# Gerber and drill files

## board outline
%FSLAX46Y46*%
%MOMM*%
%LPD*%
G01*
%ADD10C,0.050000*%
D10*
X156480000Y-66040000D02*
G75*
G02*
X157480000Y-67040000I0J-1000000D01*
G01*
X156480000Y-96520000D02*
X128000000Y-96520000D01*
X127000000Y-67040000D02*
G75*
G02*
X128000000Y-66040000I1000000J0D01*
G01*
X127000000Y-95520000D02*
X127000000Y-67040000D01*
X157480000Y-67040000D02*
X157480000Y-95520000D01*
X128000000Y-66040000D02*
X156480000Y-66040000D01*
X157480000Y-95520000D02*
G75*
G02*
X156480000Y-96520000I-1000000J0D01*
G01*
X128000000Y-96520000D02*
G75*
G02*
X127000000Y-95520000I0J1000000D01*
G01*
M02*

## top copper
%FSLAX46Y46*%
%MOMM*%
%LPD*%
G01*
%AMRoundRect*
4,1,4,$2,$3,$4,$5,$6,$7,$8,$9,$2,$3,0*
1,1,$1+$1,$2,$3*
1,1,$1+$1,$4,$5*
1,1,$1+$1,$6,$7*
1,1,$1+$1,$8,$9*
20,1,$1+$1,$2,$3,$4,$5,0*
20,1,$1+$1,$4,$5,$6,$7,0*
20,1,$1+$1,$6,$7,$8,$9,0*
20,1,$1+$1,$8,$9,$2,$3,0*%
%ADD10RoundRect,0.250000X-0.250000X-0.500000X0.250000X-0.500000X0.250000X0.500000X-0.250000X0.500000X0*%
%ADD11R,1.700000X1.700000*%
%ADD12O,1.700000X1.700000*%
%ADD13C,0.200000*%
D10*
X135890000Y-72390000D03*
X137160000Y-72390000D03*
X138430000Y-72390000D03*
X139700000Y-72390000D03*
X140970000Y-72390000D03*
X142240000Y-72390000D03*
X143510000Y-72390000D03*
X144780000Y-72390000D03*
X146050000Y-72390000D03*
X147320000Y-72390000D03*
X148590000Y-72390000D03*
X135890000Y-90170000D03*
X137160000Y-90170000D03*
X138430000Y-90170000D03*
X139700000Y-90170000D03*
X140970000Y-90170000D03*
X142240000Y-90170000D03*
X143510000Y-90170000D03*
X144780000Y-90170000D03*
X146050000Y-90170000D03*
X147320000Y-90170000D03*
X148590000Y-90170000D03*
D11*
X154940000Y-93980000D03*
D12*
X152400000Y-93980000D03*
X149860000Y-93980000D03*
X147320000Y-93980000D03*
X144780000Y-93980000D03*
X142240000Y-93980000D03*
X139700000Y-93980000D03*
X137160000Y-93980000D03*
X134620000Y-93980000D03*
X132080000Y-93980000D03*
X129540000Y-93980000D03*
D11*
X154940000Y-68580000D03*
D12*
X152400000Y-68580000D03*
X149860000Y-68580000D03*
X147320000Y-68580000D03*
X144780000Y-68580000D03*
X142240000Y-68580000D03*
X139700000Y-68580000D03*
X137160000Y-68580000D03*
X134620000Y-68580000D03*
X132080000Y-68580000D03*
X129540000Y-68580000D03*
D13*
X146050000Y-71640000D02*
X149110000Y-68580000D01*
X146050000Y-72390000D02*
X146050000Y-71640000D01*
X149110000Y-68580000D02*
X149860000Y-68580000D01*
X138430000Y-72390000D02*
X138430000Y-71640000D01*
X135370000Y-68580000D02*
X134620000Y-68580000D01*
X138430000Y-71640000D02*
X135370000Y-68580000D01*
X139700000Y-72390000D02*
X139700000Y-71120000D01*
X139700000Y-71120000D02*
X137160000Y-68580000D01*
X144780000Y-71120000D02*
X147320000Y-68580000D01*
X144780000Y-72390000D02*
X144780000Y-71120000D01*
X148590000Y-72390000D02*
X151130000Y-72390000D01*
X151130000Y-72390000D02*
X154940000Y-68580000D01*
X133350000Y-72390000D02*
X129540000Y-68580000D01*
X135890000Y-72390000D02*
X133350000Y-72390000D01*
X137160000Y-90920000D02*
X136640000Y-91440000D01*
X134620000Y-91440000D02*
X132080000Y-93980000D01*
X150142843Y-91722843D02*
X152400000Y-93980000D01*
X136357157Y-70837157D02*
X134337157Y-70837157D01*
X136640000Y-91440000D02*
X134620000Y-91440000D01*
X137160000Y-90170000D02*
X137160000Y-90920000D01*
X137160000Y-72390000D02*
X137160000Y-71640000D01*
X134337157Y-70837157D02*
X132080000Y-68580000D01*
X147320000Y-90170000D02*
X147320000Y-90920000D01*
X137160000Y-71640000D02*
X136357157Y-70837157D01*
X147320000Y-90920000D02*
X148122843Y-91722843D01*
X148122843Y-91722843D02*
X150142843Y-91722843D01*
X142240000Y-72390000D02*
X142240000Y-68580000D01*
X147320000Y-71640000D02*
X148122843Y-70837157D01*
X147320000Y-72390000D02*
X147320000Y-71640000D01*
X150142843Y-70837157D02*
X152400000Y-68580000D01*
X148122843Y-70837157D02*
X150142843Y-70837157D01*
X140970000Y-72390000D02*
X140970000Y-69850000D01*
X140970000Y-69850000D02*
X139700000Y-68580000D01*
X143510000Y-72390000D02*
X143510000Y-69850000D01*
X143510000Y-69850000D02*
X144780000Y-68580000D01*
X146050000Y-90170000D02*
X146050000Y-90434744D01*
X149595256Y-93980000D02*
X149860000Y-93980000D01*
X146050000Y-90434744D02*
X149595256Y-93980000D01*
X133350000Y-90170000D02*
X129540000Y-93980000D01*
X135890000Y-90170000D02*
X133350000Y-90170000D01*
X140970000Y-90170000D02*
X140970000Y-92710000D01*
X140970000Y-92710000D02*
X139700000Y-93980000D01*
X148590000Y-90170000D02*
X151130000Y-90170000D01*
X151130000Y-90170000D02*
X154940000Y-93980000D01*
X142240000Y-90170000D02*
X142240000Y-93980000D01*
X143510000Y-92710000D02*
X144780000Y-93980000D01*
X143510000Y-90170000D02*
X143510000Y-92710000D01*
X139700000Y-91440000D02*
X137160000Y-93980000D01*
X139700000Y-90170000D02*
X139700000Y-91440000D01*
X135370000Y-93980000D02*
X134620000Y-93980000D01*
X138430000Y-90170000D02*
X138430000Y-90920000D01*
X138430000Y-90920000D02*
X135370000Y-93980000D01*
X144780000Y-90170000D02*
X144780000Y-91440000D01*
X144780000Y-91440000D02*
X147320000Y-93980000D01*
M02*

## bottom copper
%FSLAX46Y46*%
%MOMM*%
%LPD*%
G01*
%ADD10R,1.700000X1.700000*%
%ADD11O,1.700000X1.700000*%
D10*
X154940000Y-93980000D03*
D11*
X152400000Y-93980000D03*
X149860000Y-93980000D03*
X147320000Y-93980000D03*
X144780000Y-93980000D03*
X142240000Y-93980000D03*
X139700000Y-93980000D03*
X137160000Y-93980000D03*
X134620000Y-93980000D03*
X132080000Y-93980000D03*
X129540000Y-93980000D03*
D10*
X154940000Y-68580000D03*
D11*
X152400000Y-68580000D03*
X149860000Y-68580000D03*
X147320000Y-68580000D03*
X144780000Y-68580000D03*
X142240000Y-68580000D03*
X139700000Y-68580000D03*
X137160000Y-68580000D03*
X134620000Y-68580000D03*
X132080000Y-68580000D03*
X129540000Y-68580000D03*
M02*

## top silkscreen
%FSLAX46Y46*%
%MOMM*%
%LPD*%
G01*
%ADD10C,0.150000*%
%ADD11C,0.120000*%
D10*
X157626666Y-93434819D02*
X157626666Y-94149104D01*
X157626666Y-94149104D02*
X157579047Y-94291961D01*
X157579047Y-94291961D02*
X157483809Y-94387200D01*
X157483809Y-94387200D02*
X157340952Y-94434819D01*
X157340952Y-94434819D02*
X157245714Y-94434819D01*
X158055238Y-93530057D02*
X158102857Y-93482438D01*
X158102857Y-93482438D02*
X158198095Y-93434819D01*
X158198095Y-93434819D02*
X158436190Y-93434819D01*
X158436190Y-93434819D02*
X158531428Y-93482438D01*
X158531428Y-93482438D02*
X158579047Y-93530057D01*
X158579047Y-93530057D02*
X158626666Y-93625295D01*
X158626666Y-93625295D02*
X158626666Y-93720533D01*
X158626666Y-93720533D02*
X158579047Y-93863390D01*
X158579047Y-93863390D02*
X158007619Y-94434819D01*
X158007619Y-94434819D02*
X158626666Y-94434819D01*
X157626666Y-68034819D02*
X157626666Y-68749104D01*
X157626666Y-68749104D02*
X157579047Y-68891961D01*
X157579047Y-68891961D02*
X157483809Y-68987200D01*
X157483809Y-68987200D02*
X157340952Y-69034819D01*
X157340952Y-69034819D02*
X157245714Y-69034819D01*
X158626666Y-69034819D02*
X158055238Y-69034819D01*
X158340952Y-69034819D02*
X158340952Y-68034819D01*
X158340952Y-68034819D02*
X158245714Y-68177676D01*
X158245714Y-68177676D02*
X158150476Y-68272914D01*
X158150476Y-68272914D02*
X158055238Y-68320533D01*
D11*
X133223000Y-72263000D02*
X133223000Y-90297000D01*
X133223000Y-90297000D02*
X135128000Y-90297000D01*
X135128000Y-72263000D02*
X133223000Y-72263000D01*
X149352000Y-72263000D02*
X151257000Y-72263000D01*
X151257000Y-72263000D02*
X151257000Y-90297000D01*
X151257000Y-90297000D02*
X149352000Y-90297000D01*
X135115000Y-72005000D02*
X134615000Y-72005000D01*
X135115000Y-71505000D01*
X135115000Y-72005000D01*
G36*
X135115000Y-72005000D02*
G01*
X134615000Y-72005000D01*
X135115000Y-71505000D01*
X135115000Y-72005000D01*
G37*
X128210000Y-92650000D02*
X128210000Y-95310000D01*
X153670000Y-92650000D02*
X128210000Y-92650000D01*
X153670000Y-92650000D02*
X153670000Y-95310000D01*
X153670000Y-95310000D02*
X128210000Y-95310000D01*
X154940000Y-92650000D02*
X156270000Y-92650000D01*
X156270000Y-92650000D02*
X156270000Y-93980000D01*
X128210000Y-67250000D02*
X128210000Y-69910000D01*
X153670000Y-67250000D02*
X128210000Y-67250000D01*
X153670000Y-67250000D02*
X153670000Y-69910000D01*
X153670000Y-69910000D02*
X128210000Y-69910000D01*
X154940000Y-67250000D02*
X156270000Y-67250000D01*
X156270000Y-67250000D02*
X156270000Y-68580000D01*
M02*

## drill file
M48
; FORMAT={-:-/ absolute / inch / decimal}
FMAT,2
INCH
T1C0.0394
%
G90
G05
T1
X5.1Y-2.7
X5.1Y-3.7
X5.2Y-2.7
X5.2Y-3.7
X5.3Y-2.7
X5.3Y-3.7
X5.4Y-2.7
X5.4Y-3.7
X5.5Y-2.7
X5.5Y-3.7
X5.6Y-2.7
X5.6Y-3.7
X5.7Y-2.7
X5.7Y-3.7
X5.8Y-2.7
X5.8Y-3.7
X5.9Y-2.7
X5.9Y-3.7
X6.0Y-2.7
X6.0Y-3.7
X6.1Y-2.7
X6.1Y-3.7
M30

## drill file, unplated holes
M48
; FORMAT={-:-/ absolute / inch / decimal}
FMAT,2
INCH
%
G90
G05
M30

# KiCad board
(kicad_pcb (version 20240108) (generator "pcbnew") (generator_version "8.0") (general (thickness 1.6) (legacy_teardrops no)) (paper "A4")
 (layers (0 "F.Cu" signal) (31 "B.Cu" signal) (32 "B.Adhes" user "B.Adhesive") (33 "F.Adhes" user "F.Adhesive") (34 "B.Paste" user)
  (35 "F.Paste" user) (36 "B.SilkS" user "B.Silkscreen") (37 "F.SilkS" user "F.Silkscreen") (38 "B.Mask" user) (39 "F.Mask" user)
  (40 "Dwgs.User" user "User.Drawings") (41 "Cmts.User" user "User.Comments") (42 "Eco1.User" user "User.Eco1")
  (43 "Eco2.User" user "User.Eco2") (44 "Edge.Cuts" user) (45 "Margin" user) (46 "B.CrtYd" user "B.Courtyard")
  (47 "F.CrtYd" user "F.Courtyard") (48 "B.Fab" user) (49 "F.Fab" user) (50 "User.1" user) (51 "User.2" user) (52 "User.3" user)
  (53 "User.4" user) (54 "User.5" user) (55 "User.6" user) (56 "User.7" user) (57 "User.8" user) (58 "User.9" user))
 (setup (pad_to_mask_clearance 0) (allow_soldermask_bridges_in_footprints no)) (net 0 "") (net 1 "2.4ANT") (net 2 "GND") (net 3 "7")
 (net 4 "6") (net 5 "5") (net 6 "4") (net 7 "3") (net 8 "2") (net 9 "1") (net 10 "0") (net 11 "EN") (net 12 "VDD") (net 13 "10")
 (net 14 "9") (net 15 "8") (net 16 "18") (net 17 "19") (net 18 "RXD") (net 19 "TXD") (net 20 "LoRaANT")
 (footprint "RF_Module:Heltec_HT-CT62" (layer "F.Cu") (at 142.24 81.28)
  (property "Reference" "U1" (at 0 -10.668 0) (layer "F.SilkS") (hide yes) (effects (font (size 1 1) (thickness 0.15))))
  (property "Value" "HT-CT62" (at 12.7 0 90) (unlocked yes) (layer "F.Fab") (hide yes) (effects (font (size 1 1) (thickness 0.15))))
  (fp_line (start -9.017 -9.017) (end -9.017 9.017) (stroke (width 0.12) (type default)) (layer "F.SilkS"))
  (fp_line (start -9.017 9.017) (end -7.112 9.017) (stroke (width 0.12) (type default)) (layer "F.SilkS"))
  (fp_line (start -7.112 -9.017) (end -9.017 -9.017) (stroke (width 0.12) (type default)) (layer "F.SilkS"))
  (fp_line (start 7.112 -9.017) (end 9.017 -9.017) (stroke (width 0.12) (type default)) (layer "F.SilkS"))
  (fp_line (start 9.017 -9.017) (end 9.017 9.017) (stroke (width 0.12) (type default)) (layer "F.SilkS"))
  (fp_line (start 9.017 9.017) (end 7.112 9.017) (stroke (width 0.12) (type default)) (layer "F.SilkS"))
  (fp_poly
   (pts (xy -7.125 -9.275) (xy -7.625 -9.275) (xy -7.125 -9.775) (xy -7.125 -9.275)) (stroke (width 0.12) (type solid)) (fill solid)
   (layer "F.SilkS"))
  (pad "1" smd roundrect (at -6.35 -8.89) (size 1 1.5) (layers "F.Cu" "F.Paste" "F.Mask") (roundrect_rratio 0.25) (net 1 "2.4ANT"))
  (pad "2" smd roundrect (at -5.08 -8.89) (size 1 1.5) (layers "F.Cu" "F.Paste" "F.Mask") (roundrect_rratio 0.25) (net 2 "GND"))
  (pad "3" smd roundrect (at -3.81 -8.89) (size 1 1.5) (layers "F.Cu" "F.Paste" "F.Mask") (roundrect_rratio 0.25) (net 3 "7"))
  (pad "4" smd roundrect (at -2.54 -8.89) (size 1 1.5) (layers "F.Cu" "F.Paste" "F.Mask") (roundrect_rratio 0.25) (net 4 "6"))
  (pad "5" smd roundrect (at -1.27 -8.89) (size 1 1.5) (layers "F.Cu" "F.Paste" "F.Mask") (roundrect_rratio 0.25) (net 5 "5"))
  (pad "6" smd roundrect (at 0 -8.89) (size 1 1.5) (layers "F.Cu" "F.Paste" "F.Mask") (roundrect_rratio 0.25) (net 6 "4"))
  (pad "7" smd roundrect (at 1.27 -8.89) (size 1 1.5) (layers "F.Cu" "F.Paste" "F.Mask") (roundrect_rratio 0.25) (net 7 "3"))
  (pad "8" smd roundrect (at 2.54 -8.89) (size 1 1.5) (layers "F.Cu" "F.Paste" "F.Mask") (roundrect_rratio 0.25) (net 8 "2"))
  (pad "9" smd roundrect (at 3.81 -8.89) (size 1 1.5) (layers "F.Cu" "F.Paste" "F.Mask") (roundrect_rratio 0.25) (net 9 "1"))
  (pad "10" smd roundrect (at 5.08 -8.89) (size 1 1.5) (layers "F.Cu" "F.Paste" "F.Mask") (roundrect_rratio 0.25) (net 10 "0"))
  (pad "11" smd roundrect (at 6.35 -8.89) (size 1 1.5) (layers "F.Cu" "F.Paste" "F.Mask") (roundrect_rratio 0.25) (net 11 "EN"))
  (pad "12" smd roundrect (at -6.35 8.89) (size 1 1.5) (layers "F.Cu" "F.Paste" "F.Mask") (roundrect_rratio 0.25) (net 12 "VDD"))
  (pad "13" smd roundrect (at -5.08 8.89) (size 1 1.5) (layers "F.Cu" "F.Paste" "F.Mask") (roundrect_rratio 0.25) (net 2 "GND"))
  (pad "14" smd roundrect (at -3.81 8.89) (size 1 1.5) (layers "F.Cu" "F.Paste" "F.Mask") (roundrect_rratio 0.25) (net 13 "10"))
  (pad "15" smd roundrect (at -2.54 8.89) (size 1 1.5) (layers "F.Cu" "F.Paste" "F.Mask") (roundrect_rratio 0.25) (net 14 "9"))
  (pad "16" smd roundrect (at -1.27 8.89) (size 1 1.5) (layers "F.Cu" "F.Paste" "F.Mask") (roundrect_rratio 0.25) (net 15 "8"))
  (pad "17" smd roundrect (at 0 8.89) (size 1 1.5) (layers "F.Cu" "F.Paste" "F.Mask") (roundrect_rratio 0.25) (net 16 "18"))
  (pad "18" smd roundrect (at 1.27 8.89) (size 1 1.5) (layers "F.Cu" "F.Paste" "F.Mask") (roundrect_rratio 0.25) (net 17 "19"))
  (pad "19" smd roundrect (at 2.54 8.89) (size 1 1.5) (layers "F.Cu" "F.Paste" "F.Mask") (roundrect_rratio 0.25) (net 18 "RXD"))
  (pad "20" smd roundrect (at 3.81 8.89) (size 1 1.5) (layers "F.Cu" "F.Paste" "F.Mask") (roundrect_rratio 0.25) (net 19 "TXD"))
  (pad "21" smd roundrect (at 5.08 8.89) (size 1 1.5) (layers "F.Cu" "F.Paste" "F.Mask") (roundrect_rratio 0.25) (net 2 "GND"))
  (pad "22" smd roundrect (at 6.35 8.89) (size 1 1.5) (layers "F.Cu" "F.Paste" "F.Mask") (roundrect_rratio 0.25) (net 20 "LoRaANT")))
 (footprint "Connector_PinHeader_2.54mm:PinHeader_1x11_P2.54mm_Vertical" (layer "F.Cu") (at 154.94 93.98 -90)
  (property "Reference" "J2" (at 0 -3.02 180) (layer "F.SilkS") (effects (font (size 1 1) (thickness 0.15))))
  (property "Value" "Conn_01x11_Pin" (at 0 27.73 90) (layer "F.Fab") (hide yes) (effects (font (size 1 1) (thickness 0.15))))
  (fp_line (start -1.33 26.73) (end 1.33 26.73) (stroke (width 0.12) (type solid)) (layer "F.SilkS"))
  (fp_line (start -1.33 1.27) (end -1.33 26.73) (stroke (width 0.12) (type solid)) (layer "F.SilkS"))
  (fp_line (start -1.33 1.27) (end 1.33 1.27) (stroke (width 0.12) (type solid)) (layer "F.SilkS"))
  (fp_line (start 1.33 1.27) (end 1.33 26.73) (stroke (width 0.12) (type solid)) (layer "F.SilkS"))
  (fp_line (start -1.33 0) (end -1.33 -1.33) (stroke (width 0.12) (type solid)) (layer "F.SilkS"))
  (fp_line (start -1.33 -1.33) (end 0 -1.33) (stroke (width 0.12) (type solid)) (layer "F.SilkS"))
  (pad "1" thru_hole rect (at 0 0 270) (size 1.7 1.7) (drill 1) (layers "*.Cu" "*.Mask") (remove_unused_layers no) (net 20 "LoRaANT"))
  (pad "2" thru_hole oval (at 0 2.54 270) (size 1.7 1.7) (drill 1) (layers "*.Cu" "*.Mask") (remove_unused_layers no) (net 2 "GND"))
  (pad "3" thru_hole oval (at 0 5.08 270) (size 1.7 1.7) (drill 1) (layers "*.Cu" "*.Mask") (remove_unused_layers no) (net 19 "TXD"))
  (pad "4" thru_hole oval (at 0 7.62 270) (size 1.7 1.7) (drill 1) (layers "*.Cu" "*.Mask") (remove_unused_layers no) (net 18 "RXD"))
  (pad "5" thru_hole oval (at 0 10.16 270) (size 1.7 1.7) (drill 1) (layers "*.Cu" "*.Mask") (remove_unused_layers no) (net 17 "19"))
  (pad "6" thru_hole oval (at 0 12.7 270) (size 1.7 1.7) (drill 1) (layers "*.Cu" "*.Mask") (remove_unused_layers no) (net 16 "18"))
  (pad "7" thru_hole oval (at 0 15.24 270) (size 1.7 1.7) (drill 1) (layers "*.Cu" "*.Mask") (remove_unused_layers no) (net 15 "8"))
  (pad "8" thru_hole oval (at 0 17.78 270) (size 1.7 1.7) (drill 1) (layers "*.Cu" "*.Mask") (remove_unused_layers no) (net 14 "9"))
  (pad "9" thru_hole oval (at 0 20.32 270) (size 1.7 1.7) (drill 1) (layers "*.Cu" "*.Mask") (remove_unused_layers no) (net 13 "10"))
  (pad "10" thru_hole oval (at 0 22.86 270) (size 1.7 1.7) (drill 1) (layers "*.Cu" "*.Mask") (remove_unused_layers no) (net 2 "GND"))
  (pad "11" thru_hole oval (at 0 25.4 270) (size 1.7 1.7) (drill 1) (layers "*.Cu" "*.Mask") (remove_unused_layers no) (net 12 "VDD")))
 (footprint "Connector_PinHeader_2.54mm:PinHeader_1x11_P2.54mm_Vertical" (layer "F.Cu") (at 154.94 68.58 -90)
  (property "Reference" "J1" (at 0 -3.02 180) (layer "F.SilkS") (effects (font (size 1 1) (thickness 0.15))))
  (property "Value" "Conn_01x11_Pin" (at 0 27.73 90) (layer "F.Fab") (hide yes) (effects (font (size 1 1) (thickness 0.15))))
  (fp_line (start -1.33 26.73) (end 1.33 26.73) (stroke (width 0.12) (type solid)) (layer "F.SilkS"))
  (fp_line (start -1.33 1.27) (end -1.33 26.73) (stroke (width 0.12) (type solid)) (layer "F.SilkS"))
  (fp_line (start -1.33 1.27) (end 1.33 1.27) (stroke (width 0.12) (type solid)) (layer "F.SilkS"))
  (fp_line (start 1.33 1.27) (end 1.33 26.73) (stroke (width 0.12) (type solid)) (layer "F.SilkS"))
  (fp_line (start -1.33 0) (end -1.33 -1.33) (stroke (width 0.12) (type solid)) (layer "F.SilkS"))
  (fp_line (start -1.33 -1.33) (end 0 -1.33) (stroke (width 0.12) (type solid)) (layer "F.SilkS"))
  (pad "1" thru_hole rect (at 0 0 270) (size 1.7 1.7) (drill 1) (layers "*.Cu" "*.Mask") (remove_unused_layers no) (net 11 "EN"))
  (pad "2" thru_hole oval (at 0 2.54 270) (size 1.7 1.7) (drill 1) (layers "*.Cu" "*.Mask") (remove_unused_layers no) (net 10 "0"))
  (pad "3" thru_hole oval (at 0 5.08 270) (size 1.7 1.7) (drill 1) (layers "*.Cu" "*.Mask") (remove_unused_layers no) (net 9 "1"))
  (pad "4" thru_hole oval (at 0 7.62 270) (size 1.7 1.7) (drill 1) (layers "*.Cu" "*.Mask") (remove_unused_layers no) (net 8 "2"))
  (pad "5" thru_hole oval (at 0 10.16 270) (size 1.7 1.7) (drill 1) (layers "*.Cu" "*.Mask") (remove_unused_layers no) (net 7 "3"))
  (pad "6" thru_hole oval (at 0 12.7 270) (size 1.7 1.7) (drill 1) (layers "*.Cu" "*.Mask") (remove_unused_layers no) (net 6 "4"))
  (pad "7" thru_hole oval (at 0 15.24 270) (size 1.7 1.7) (drill 1) (layers "*.Cu" "*.Mask") (remove_unused_layers no) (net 5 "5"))
  (pad "8" thru_hole oval (at 0 17.78 270) (size 1.7 1.7) (drill 1) (layers "*.Cu" "*.Mask") (remove_unused_layers no) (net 4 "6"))
  (pad "9" thru_hole oval (at 0 20.32 270) (size 1.7 1.7) (drill 1) (layers "*.Cu" "*.Mask") (remove_unused_layers no) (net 3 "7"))
  (pad "10" thru_hole oval (at 0 22.86 270) (size 1.7 1.7) (drill 1) (layers "*.Cu" "*.Mask") (remove_unused_layers no) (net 2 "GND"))
  (pad "11" thru_hole oval (at 0 25.4 270) (size 1.7 1.7) (drill 1) (layers "*.Cu" "*.Mask") (remove_unused_layers no) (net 1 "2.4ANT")))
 (gr_arc (start 156.48 66.04) (mid 157.187107 66.332893) (end 157.48 67.04) (stroke (width 0.05) (type default)) (layer "Edge.Cuts"))
 (gr_line (start 156.48 96.52) (end 128 96.52) (stroke (width 0.05) (type default)) (layer "Edge.Cuts"))
 (gr_arc (start 127 67.04) (mid 127.292893 66.332893) (end 128 66.04) (stroke (width 0.05) (type default)) (layer "Edge.Cuts"))
 (gr_line (start 127 95.52) (end 127 67.04) (stroke (width 0.05) (type default)) (layer "Edge.Cuts"))
 (gr_line (start 157.48 67.04) (end 157.48 95.52) (stroke (width 0.05) (type default)) (layer "Edge.Cuts"))
 (gr_line (start 128 66.04) (end 156.48 66.04) (stroke (width 0.05) (type default)) (layer "Edge.Cuts"))
 (gr_arc (start 157.48 95.52) (mid 157.187107 96.227107) (end 156.48 96.52) (stroke (width 0.05) (type default)) (layer "Edge.Cuts"))
 (gr_arc (start 128 96.52) (mid 127.292893 96.227107) (end 127 95.52) (stroke (width 0.05) (type default)) (layer "Edge.Cuts"))
 (segment (start 146.05 71.64) (end 149.11 68.58) (width 0.2) (layer "F.Cu") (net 9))
 (segment (start 146.05 72.39) (end 146.05 71.64) (width 0.2) (layer "F.Cu") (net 9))
 (segment (start 149.11 68.58) (end 149.86 68.58) (width 0.2) (layer "F.Cu") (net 9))
 (segment (start 138.43 72.39) (end 138.43 71.64) (width 0.2) (layer "F.Cu") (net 3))
 (segment (start 135.37 68.58) (end 134.62 68.58) (width 0.2) (layer "F.Cu") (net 3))
 (segment (start 138.43 71.64) (end 135.37 68.58) (width 0.2) (layer "F.Cu") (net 3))
 (segment (start 139.7 72.39) (end 139.7 71.12) (width 0.2) (layer "F.Cu") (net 4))
 (segment (start 139.7 71.12) (end 137.16 68.58) (width 0.2) (layer "F.Cu") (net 4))
 (segment (start 144.78 71.12) (end 147.32 68.58) (width 0.2) (layer "F.Cu") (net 8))
 (segment (start 144.78 72.39) (end 144.78 71.12) (width 0.2) (layer "F.Cu") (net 8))
 (segment (start 148.59 72.39) (end 151.13 72.39) (width 0.2) (layer "F.Cu") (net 11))
 (segment (start 151.13 72.39) (end 154.94 68.58) (width 0.2) (layer "F.Cu") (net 11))
 (segment (start 133.35 72.39) (end 129.54 68.58) (width 0.2) (layer "F.Cu") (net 1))
 (segment (start 135.89 72.39) (end 133.35 72.39) (width 0.2) (layer "F.Cu") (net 1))
 (segment (start 137.16 90.92) (end 136.64 91.44) (width 0.2) (layer "F.Cu") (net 2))
 (segment (start 134.62 91.44) (end 132.08 93.98) (width 0.2) (layer "F.Cu") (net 2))
 (segment (start 150.142843 91.722843) (end 152.4 93.98) (width 0.2) (layer "F.Cu") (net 2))
 (segment (start 136.357157 70.837157) (end 134.337157 70.837157) (width 0.2) (layer "F.Cu") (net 2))
 (segment (start 136.64 91.44) (end 134.62 91.44) (width 0.2) (layer "F.Cu") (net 2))
 (segment (start 137.16 90.17) (end 137.16 90.92) (width 0.2) (layer "F.Cu") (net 2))
 (segment (start 137.16 72.39) (end 137.16 71.64) (width 0.2) (layer "F.Cu") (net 2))
 (segment (start 134.337157 70.837157) (end 132.08 68.58) (width 0.2) (layer "F.Cu") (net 2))
 (segment (start 147.32 90.17) (end 147.32 90.92) (width 0.2) (layer "F.Cu") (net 2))
 (segment (start 137.16 71.64) (end 136.357157 70.837157) (width 0.2) (layer "F.Cu") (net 2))
 (segment (start 147.32 90.92) (end 148.122843 91.722843) (width 0.2) (layer "F.Cu") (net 2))
 (segment (start 148.122843 91.722843) (end 150.142843 91.722843) (width 0.2) (layer "F.Cu") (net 2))
 (segment (start 142.24 72.39) (end 142.24 68.58) (width 0.2) (layer "F.Cu") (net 6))
 (segment (start 147.32 71.64) (end 148.122843 70.837157) (width 0.2) (layer "F.Cu") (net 10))
 (segment (start 147.32 72.39) (end 147.32 71.64) (width 0.2) (layer "F.Cu") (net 10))
 (segment (start 150.142843 70.837157) (end 152.4 68.58) (width 0.2) (layer "F.Cu") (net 10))
 (segment (start 148.122843 70.837157) (end 150.142843 70.837157) (width 0.2) (layer "F.Cu") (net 10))
 (segment (start 140.97 72.39) (end 140.97 69.85) (width 0.2) (layer "F.Cu") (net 5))
 (segment (start 140.97 69.85) (end 139.7 68.58) (width 0.2) (layer "F.Cu") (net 5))
 (segment (start 143.51 72.39) (end 143.51 69.85) (width 0.2) (layer "F.Cu") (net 7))
 (segment (start 143.51 69.85) (end 144.78 68.58) (width 0.2) (layer "F.Cu") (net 7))
 (segment (start 146.05 90.17) (end 146.05 90.434744) (width 0.2) (layer "F.Cu") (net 19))
 (segment (start 149.595256 93.98) (end 149.86 93.98) (width 0.2) (layer "F.Cu") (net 19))
 (segment (start 146.05 90.434744) (end 149.595256 93.98) (width 0.2) (layer "F.Cu") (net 19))
 (segment (start 133.35 90.17) (end 129.54 93.98) (width 0.2) (layer "F.Cu") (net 12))
 (segment (start 135.89 90.17) (end 133.35 90.17) (width 0.2) (layer "F.Cu") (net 12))
 (segment (start 140.97 90.17) (end 140.97 92.71) (width 0.2) (layer "F.Cu") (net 15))
 (segment (start 140.97 92.71) (end 139.7 93.98) (width 0.2) (layer "F.Cu") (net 15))
 (segment (start 148.59 90.17) (end 151.13 90.17) (width 0.2) (layer "F.Cu") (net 20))
 (segment (start 151.13 90.17) (end 154.94 93.98) (width 0.2) (layer "F.Cu") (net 20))
 (segment (start 142.24 90.17) (end 142.24 93.98) (width 0.2) (layer "F.Cu") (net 16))
 (segment (start 143.51 92.71) (end 144.78 93.98) (width 0.2) (layer "F.Cu") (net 17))
 (segment (start 143.51 90.17) (end 143.51 92.71) (width 0.2) (layer "F.Cu") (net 17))
 (segment (start 139.7 91.44) (end 137.16 93.98) (width 0.2) (layer "F.Cu") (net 14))
 (segment (start 139.7 90.17) (end 139.7 91.44) (width 0.2) (layer "F.Cu") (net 14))
 (segment (start 135.37 93.98) (end 134.62 93.98) (width 0.2) (layer "F.Cu") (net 13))
 (segment (start 138.43 90.17) (end 138.43 90.92) (width 0.2) (layer "F.Cu") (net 13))
 (segment (start 138.43 90.92) (end 135.37 93.98) (width 0.2) (layer "F.Cu") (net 13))
 (segment (start 144.78 90.17) (end 144.78 91.44) (width 0.2) (layer "F.Cu") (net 18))
 (segment (start 144.78 91.44) (end 147.32 93.98) (width 0.2) (layer "F.Cu") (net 18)))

